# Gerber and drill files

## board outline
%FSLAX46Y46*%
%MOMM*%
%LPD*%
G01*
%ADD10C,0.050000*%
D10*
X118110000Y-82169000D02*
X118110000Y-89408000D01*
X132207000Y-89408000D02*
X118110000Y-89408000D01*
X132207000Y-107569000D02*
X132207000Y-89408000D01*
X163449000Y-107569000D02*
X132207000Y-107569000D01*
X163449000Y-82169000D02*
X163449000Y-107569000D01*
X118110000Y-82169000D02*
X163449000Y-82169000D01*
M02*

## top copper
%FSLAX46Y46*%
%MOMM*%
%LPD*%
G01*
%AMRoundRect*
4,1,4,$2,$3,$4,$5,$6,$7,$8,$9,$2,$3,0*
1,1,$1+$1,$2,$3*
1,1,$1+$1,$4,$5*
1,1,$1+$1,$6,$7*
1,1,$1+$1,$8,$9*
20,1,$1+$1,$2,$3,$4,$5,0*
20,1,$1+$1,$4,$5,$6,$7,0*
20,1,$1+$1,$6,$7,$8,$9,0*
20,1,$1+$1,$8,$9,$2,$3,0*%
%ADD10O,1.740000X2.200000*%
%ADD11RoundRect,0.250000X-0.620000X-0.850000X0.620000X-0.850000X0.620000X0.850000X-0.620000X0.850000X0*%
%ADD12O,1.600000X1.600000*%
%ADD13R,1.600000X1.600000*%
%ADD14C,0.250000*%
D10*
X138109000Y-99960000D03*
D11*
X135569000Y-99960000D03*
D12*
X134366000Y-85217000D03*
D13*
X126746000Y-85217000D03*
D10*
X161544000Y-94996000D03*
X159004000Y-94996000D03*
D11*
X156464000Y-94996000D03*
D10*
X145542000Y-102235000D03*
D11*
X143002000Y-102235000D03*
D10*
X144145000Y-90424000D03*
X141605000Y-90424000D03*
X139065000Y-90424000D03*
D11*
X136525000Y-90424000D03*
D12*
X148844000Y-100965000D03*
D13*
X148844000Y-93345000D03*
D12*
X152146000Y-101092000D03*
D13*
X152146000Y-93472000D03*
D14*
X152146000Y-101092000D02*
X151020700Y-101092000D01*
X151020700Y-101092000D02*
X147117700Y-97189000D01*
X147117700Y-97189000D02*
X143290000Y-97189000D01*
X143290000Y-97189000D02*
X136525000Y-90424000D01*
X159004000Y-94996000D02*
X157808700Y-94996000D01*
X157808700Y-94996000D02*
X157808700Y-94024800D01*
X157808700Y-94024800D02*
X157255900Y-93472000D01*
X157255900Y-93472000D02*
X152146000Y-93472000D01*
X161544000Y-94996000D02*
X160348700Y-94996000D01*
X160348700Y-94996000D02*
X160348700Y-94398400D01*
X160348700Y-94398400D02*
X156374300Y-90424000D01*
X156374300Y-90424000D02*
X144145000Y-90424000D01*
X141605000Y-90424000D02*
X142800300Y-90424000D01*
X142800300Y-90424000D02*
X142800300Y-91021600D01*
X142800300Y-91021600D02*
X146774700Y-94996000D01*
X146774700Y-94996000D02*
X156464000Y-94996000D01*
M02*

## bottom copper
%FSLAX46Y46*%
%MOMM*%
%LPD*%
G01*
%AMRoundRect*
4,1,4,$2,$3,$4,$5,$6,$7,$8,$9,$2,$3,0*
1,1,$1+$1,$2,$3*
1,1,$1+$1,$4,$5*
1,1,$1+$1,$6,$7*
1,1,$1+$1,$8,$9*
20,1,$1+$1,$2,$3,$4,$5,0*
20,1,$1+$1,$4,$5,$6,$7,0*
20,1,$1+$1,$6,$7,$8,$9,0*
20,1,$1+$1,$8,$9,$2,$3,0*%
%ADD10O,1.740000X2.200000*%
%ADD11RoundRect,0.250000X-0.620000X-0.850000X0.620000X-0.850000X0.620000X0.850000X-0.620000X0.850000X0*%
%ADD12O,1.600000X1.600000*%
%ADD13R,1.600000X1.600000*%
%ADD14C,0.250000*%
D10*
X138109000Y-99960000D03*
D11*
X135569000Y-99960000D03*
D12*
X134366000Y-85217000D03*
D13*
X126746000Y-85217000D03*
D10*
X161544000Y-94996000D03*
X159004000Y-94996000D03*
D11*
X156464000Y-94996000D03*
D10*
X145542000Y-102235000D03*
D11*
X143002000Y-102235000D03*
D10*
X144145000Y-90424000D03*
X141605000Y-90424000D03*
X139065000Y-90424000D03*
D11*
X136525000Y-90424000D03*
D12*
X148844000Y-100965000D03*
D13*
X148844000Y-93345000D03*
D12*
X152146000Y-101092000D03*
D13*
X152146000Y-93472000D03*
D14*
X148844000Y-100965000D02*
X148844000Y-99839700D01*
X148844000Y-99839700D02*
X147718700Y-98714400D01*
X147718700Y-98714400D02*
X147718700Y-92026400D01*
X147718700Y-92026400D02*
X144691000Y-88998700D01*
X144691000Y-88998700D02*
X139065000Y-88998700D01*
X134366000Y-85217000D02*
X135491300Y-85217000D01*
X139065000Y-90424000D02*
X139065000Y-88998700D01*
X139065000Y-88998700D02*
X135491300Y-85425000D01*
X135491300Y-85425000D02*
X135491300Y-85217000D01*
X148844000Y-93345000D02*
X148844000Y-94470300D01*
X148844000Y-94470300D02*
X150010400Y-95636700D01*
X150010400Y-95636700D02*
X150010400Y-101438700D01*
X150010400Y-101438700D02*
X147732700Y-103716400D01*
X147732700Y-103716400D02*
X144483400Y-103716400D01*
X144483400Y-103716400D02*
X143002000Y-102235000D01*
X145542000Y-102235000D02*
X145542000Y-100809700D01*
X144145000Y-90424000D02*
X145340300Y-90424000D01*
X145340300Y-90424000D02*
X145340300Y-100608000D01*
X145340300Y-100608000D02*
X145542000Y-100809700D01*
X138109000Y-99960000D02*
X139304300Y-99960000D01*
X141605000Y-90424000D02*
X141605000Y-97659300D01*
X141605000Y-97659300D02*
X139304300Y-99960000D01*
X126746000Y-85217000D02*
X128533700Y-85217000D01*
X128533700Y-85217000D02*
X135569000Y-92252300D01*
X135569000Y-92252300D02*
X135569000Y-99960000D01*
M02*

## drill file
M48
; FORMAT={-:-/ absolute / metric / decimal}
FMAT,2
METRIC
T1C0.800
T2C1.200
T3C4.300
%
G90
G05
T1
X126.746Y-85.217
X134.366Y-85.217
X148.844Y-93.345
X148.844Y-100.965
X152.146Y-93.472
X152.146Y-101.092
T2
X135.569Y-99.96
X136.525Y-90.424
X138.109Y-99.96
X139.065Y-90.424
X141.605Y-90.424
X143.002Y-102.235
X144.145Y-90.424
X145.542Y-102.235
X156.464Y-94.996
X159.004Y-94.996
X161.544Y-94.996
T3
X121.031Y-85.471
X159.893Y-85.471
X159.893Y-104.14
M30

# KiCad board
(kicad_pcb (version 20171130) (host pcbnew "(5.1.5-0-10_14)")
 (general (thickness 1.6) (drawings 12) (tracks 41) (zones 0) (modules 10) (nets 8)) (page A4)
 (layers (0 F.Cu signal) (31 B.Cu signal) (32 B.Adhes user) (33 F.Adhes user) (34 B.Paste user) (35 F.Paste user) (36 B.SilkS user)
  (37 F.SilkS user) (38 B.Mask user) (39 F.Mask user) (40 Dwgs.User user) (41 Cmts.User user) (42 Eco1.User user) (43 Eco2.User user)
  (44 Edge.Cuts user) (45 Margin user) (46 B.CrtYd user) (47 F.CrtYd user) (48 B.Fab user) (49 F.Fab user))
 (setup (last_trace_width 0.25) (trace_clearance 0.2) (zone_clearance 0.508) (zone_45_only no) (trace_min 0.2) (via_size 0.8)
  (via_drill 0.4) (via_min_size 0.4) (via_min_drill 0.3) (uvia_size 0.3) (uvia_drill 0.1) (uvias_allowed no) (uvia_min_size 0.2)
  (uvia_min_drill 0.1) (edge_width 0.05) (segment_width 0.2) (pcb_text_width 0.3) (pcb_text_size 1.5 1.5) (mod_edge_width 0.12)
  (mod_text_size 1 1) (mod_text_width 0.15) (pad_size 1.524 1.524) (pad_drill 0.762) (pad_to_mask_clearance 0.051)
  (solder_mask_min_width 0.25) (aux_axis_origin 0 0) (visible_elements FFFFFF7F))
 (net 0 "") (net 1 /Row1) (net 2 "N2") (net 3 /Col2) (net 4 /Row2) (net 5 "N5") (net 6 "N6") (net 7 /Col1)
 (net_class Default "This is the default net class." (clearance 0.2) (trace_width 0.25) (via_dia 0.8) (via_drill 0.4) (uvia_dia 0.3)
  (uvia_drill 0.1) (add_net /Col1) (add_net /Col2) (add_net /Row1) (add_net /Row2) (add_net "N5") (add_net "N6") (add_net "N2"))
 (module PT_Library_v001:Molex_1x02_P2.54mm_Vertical (layer F.Cu) (at 135.569 99.96)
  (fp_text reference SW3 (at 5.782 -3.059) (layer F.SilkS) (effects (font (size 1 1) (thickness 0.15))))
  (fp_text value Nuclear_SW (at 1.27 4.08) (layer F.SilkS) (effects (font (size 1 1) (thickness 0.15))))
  (pad 2 thru_hole oval (at 2.54 0) (size 1.74 2.2) (drill 1.2) (layers *.Cu *.Mask) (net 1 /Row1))
  (pad 1 thru_hole roundrect (at 0 0) (size 1.74 2.2) (drill 1.2) (layers *.Cu *.Mask) (roundrect_rratio 0.143678) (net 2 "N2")))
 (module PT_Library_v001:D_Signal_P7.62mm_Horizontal (layer F.Cu) (at 126.746 85.217)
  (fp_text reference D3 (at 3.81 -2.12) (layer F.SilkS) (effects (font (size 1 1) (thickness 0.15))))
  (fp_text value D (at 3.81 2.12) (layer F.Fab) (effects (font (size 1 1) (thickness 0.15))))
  (pad 2 thru_hole oval (at 7.62 0) (size 1.6 1.6) (drill 0.8) (layers *.Cu *.Mask) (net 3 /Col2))
  (pad 1 thru_hole rect (at 0 0) (size 1.6 1.6) (drill 0.8) (layers *.Cu *.Mask) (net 2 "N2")))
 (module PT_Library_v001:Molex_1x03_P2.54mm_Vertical (layer F.Cu) (at 156.464 94.996)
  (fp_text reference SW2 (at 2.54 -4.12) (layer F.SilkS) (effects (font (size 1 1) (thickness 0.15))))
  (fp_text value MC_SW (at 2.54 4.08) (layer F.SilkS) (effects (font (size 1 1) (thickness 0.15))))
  (pad 3 thru_hole oval (at 5.08 0) (size 1.74 2.2) (drill 1.2) (layers *.Cu *.Mask) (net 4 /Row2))
  (pad 2 thru_hole oval (at 2.54 0) (size 1.74 2.2) (drill 1.2) (layers *.Cu *.Mask) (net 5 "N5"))
  (pad 1 thru_hole roundrect (at 0 0) (size 1.74 2.2) (drill 1.2) (layers *.Cu *.Mask) (roundrect_rratio 0.143678) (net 1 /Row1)))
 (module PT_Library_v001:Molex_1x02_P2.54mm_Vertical (layer F.Cu) (at 143.002 102.235)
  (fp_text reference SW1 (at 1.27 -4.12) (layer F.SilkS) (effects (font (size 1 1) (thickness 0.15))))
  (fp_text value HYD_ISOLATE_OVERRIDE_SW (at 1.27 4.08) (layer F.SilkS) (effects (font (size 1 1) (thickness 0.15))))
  (pad 2 thru_hole oval (at 2.54 0) (size 1.74 2.2) (drill 1.2) (layers *.Cu *.Mask) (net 4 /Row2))
  (pad 1 thru_hole roundrect (at 0 0) (size 1.74 2.2) (drill 1.2) (layers *.Cu *.Mask) (roundrect_rratio 0.143678) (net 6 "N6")))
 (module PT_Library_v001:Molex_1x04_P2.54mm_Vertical (layer F.Cu) (at 136.525 90.424)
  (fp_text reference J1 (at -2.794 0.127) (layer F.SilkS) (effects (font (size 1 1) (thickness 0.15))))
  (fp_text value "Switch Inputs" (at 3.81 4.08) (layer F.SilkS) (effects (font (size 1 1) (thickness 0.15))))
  (pad 4 thru_hole oval (at 7.62 0) (size 1.74 2.2) (drill 1.2) (layers *.Cu *.Mask) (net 4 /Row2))
  (pad 3 thru_hole oval (at 5.08 0) (size 1.74 2.2) (drill 1.2) (layers *.Cu *.Mask) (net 1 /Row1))
  (pad 2 thru_hole oval (at 2.54 0) (size 1.74 2.2) (drill 1.2) (layers *.Cu *.Mask) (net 3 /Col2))
  (pad 1 thru_hole roundrect (at 0 0) (size 1.74 2.2) (drill 1.2) (layers *.Cu *.Mask) (roundrect_rratio 0.143678) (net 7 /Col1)))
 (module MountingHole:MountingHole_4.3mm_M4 (layer F.Cu) (at 159.893 85.471)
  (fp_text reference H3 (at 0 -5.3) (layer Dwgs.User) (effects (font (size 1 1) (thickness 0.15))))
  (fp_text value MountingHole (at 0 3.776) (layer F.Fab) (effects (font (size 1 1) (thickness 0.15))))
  (pad 1 np_thru_hole circle (at 0 0) (size 4.3 4.3) (drill 4.3) (layers *.Cu *.Mask)))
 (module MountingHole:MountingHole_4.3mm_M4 (layer F.Cu) (at 159.893 104.14)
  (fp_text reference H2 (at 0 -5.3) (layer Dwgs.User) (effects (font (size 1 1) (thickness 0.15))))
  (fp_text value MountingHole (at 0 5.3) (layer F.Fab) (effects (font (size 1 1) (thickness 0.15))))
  (pad 1 np_thru_hole circle (at 0 0) (size 4.3 4.3) (drill 4.3) (layers *.Cu *.Mask)))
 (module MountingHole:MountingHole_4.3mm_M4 (layer F.Cu) (at 121.031 85.471)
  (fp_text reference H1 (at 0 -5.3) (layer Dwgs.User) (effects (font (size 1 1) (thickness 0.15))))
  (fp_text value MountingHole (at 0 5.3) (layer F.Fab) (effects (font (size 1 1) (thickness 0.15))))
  (pad 1 np_thru_hole circle (at 0 0) (size 4.3 4.3) (drill 4.3) (layers *.Cu *.Mask)))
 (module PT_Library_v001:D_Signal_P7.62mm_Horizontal (layer F.Cu) (at 148.844 93.345 270)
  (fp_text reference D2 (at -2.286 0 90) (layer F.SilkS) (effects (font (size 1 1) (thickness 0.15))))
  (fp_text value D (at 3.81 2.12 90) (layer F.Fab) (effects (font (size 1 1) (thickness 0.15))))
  (pad 2 thru_hole oval (at 7.62 0 270) (size 1.6 1.6) (drill 0.8) (layers *.Cu *.Mask) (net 3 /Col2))
  (pad 1 thru_hole rect (at 0 0 270) (size 1.6 1.6) (drill 0.8) (layers *.Cu *.Mask) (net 6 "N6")))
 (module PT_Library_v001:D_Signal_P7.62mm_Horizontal (layer F.Cu) (at 152.146 93.472 270)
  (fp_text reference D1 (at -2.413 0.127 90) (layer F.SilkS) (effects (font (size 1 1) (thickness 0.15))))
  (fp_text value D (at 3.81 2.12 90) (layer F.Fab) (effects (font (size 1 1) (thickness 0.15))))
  (pad 2 thru_hole oval (at 7.62 0 270) (size 1.6 1.6) (drill 0.8) (layers *.Cu *.Mask) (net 7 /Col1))
  (pad 1 thru_hole rect (at 0 0 270) (size 1.6 1.6) (drill 0.8) (layers *.Cu *.Mask) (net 5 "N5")))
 (gr_line (start 118.11 82.169) (end 118.11 89.408) (layer Edge.Cuts) (width 0.05))
 (gr_line (start 132.207 89.408) (end 118.11 89.408) (layer Edge.Cuts) (width 0.05))
 (gr_line (start 132.207 107.569) (end 132.207 89.408) (layer Edge.Cuts) (width 0.05))
 (gr_line (start 163.449 107.569) (end 132.207 107.569) (layer Edge.Cuts) (width 0.05))
 (gr_line (start 163.449 82.169) (end 163.449 107.569) (layer Edge.Cuts) (width 0.05))
 (gr_line (start 118.11 82.169) (end 163.449 82.169) (layer Edge.Cuts) (width 0.05))
 (segment (start 152.146 101.092) (end 151.0207 101.092) (width 0.25) (layer F.Cu) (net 7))
 (segment (start 151.0207 101.092) (end 147.1177 97.189) (width 0.25) (layer F.Cu) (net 7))
 (segment (start 147.1177 97.189) (end 143.29 97.189) (width 0.25) (layer F.Cu) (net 7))
 (segment (start 143.29 97.189) (end 136.525 90.424) (width 0.25) (layer F.Cu) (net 7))
 (segment (start 159.004 94.996) (end 157.8087 94.996) (width 0.25) (layer F.Cu) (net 5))
 (segment (start 157.8087 94.996) (end 157.8087 94.0248) (width 0.25) (layer F.Cu) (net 5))
 (segment (start 157.8087 94.0248) (end 157.2559 93.472) (width 0.25) (layer F.Cu) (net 5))
 (segment (start 157.2559 93.472) (end 152.146 93.472) (width 0.25) (layer F.Cu) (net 5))
 (segment (start 148.844 100.965) (end 148.844 99.8397) (width 0.25) (layer B.Cu) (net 3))
 (segment (start 148.844 99.8397) (end 147.7187 98.7144) (width 0.25) (layer B.Cu) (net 3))
 (segment (start 147.7187 98.7144) (end 147.7187 92.0264) (width 0.25) (layer B.Cu) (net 3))
 (segment (start 147.7187 92.0264) (end 144.691 88.9987) (width 0.25) (layer B.Cu) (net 3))
 (segment (start 144.691 88.9987) (end 139.065 88.9987) (width 0.25) (layer B.Cu) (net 3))
 (segment (start 134.366 85.217) (end 135.4913 85.217) (width 0.25) (layer B.Cu) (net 3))
 (segment (start 139.065 90.424) (end 139.065 88.9987) (width 0.25) (layer B.Cu) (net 3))
 (segment (start 139.065 88.9987) (end 135.4913 85.425) (width 0.25) (layer B.Cu) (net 3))
 (segment (start 135.4913 85.425) (end 135.4913 85.217) (width 0.25) (layer B.Cu) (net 3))
 (segment (start 148.844 93.345) (end 148.844 94.4703) (width 0.25) (layer B.Cu) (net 6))
 (segment (start 148.844 94.4703) (end 150.0104 95.6367) (width 0.25) (layer B.Cu) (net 6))
 (segment (start 150.0104 95.6367) (end 150.0104 101.4387) (width 0.25) (layer B.Cu) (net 6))
 (segment (start 150.0104 101.4387) (end 147.7327 103.7164) (width 0.25) (layer B.Cu) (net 6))
 (segment (start 147.7327 103.7164) (end 144.4834 103.7164) (width 0.25) (layer B.Cu) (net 6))
 (segment (start 144.4834 103.7164) (end 143.002 102.235) (width 0.25) (layer B.Cu) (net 6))
 (segment (start 161.544 94.996) (end 160.3487 94.996) (width 0.25) (layer F.Cu) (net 4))
 (segment (start 160.3487 94.996) (end 160.3487 94.3984) (width 0.25) (layer F.Cu) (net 4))
 (segment (start 160.3487 94.3984) (end 156.3743 90.424) (width 0.25) (layer F.Cu) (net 4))
 (segment (start 156.3743 90.424) (end 144.145 90.424) (width 0.25) (layer F.Cu) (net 4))
 (segment (start 145.542 102.235) (end 145.542 100.8097) (width 0.25) (layer B.Cu) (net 4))
 (segment (start 144.145 90.424) (end 145.3403 90.424) (width 0.25) (layer B.Cu) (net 4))
 (segment (start 145.3403 90.424) (end 145.3403 100.608) (width 0.25) (layer B.Cu) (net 4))
 (segment (start 145.3403 100.608) (end 145.542 100.8097) (width 0.25) (layer B.Cu) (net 4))
 (segment (start 138.109 99.96) (end 139.3043 99.96) (width 0.25) (layer B.Cu) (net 1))
 (segment (start 141.605 90.424) (end 141.605 97.6593) (width 0.25) (layer B.Cu) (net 1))
 (segment (start 141.605 97.6593) (end 139.3043 99.96) (width 0.25) (layer B.Cu) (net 1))
 (segment (start 141.605 90.424) (end 142.8003 90.424) (width 0.25) (layer F.Cu) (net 1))
 (segment (start 142.8003 90.424) (end 142.8003 91.0216) (width 0.25) (layer F.Cu) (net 1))
 (segment (start 142.8003 91.0216) (end 146.7747 94.996) (width 0.25) (layer F.Cu) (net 1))
 (segment (start 146.7747 94.996) (end 156.464 94.996) (width 0.25) (layer F.Cu) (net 1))
 (segment (start 126.746 85.217) (end 128.5337 85.217) (width 0.25) (layer B.Cu) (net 2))
 (segment (start 128.5337 85.217) (end 135.569 92.2523) (width 0.25) (layer B.Cu) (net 2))
 (segment (start 135.569 92.2523) (end 135.569 99.96) (width 0.25) (layer B.Cu) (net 2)))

